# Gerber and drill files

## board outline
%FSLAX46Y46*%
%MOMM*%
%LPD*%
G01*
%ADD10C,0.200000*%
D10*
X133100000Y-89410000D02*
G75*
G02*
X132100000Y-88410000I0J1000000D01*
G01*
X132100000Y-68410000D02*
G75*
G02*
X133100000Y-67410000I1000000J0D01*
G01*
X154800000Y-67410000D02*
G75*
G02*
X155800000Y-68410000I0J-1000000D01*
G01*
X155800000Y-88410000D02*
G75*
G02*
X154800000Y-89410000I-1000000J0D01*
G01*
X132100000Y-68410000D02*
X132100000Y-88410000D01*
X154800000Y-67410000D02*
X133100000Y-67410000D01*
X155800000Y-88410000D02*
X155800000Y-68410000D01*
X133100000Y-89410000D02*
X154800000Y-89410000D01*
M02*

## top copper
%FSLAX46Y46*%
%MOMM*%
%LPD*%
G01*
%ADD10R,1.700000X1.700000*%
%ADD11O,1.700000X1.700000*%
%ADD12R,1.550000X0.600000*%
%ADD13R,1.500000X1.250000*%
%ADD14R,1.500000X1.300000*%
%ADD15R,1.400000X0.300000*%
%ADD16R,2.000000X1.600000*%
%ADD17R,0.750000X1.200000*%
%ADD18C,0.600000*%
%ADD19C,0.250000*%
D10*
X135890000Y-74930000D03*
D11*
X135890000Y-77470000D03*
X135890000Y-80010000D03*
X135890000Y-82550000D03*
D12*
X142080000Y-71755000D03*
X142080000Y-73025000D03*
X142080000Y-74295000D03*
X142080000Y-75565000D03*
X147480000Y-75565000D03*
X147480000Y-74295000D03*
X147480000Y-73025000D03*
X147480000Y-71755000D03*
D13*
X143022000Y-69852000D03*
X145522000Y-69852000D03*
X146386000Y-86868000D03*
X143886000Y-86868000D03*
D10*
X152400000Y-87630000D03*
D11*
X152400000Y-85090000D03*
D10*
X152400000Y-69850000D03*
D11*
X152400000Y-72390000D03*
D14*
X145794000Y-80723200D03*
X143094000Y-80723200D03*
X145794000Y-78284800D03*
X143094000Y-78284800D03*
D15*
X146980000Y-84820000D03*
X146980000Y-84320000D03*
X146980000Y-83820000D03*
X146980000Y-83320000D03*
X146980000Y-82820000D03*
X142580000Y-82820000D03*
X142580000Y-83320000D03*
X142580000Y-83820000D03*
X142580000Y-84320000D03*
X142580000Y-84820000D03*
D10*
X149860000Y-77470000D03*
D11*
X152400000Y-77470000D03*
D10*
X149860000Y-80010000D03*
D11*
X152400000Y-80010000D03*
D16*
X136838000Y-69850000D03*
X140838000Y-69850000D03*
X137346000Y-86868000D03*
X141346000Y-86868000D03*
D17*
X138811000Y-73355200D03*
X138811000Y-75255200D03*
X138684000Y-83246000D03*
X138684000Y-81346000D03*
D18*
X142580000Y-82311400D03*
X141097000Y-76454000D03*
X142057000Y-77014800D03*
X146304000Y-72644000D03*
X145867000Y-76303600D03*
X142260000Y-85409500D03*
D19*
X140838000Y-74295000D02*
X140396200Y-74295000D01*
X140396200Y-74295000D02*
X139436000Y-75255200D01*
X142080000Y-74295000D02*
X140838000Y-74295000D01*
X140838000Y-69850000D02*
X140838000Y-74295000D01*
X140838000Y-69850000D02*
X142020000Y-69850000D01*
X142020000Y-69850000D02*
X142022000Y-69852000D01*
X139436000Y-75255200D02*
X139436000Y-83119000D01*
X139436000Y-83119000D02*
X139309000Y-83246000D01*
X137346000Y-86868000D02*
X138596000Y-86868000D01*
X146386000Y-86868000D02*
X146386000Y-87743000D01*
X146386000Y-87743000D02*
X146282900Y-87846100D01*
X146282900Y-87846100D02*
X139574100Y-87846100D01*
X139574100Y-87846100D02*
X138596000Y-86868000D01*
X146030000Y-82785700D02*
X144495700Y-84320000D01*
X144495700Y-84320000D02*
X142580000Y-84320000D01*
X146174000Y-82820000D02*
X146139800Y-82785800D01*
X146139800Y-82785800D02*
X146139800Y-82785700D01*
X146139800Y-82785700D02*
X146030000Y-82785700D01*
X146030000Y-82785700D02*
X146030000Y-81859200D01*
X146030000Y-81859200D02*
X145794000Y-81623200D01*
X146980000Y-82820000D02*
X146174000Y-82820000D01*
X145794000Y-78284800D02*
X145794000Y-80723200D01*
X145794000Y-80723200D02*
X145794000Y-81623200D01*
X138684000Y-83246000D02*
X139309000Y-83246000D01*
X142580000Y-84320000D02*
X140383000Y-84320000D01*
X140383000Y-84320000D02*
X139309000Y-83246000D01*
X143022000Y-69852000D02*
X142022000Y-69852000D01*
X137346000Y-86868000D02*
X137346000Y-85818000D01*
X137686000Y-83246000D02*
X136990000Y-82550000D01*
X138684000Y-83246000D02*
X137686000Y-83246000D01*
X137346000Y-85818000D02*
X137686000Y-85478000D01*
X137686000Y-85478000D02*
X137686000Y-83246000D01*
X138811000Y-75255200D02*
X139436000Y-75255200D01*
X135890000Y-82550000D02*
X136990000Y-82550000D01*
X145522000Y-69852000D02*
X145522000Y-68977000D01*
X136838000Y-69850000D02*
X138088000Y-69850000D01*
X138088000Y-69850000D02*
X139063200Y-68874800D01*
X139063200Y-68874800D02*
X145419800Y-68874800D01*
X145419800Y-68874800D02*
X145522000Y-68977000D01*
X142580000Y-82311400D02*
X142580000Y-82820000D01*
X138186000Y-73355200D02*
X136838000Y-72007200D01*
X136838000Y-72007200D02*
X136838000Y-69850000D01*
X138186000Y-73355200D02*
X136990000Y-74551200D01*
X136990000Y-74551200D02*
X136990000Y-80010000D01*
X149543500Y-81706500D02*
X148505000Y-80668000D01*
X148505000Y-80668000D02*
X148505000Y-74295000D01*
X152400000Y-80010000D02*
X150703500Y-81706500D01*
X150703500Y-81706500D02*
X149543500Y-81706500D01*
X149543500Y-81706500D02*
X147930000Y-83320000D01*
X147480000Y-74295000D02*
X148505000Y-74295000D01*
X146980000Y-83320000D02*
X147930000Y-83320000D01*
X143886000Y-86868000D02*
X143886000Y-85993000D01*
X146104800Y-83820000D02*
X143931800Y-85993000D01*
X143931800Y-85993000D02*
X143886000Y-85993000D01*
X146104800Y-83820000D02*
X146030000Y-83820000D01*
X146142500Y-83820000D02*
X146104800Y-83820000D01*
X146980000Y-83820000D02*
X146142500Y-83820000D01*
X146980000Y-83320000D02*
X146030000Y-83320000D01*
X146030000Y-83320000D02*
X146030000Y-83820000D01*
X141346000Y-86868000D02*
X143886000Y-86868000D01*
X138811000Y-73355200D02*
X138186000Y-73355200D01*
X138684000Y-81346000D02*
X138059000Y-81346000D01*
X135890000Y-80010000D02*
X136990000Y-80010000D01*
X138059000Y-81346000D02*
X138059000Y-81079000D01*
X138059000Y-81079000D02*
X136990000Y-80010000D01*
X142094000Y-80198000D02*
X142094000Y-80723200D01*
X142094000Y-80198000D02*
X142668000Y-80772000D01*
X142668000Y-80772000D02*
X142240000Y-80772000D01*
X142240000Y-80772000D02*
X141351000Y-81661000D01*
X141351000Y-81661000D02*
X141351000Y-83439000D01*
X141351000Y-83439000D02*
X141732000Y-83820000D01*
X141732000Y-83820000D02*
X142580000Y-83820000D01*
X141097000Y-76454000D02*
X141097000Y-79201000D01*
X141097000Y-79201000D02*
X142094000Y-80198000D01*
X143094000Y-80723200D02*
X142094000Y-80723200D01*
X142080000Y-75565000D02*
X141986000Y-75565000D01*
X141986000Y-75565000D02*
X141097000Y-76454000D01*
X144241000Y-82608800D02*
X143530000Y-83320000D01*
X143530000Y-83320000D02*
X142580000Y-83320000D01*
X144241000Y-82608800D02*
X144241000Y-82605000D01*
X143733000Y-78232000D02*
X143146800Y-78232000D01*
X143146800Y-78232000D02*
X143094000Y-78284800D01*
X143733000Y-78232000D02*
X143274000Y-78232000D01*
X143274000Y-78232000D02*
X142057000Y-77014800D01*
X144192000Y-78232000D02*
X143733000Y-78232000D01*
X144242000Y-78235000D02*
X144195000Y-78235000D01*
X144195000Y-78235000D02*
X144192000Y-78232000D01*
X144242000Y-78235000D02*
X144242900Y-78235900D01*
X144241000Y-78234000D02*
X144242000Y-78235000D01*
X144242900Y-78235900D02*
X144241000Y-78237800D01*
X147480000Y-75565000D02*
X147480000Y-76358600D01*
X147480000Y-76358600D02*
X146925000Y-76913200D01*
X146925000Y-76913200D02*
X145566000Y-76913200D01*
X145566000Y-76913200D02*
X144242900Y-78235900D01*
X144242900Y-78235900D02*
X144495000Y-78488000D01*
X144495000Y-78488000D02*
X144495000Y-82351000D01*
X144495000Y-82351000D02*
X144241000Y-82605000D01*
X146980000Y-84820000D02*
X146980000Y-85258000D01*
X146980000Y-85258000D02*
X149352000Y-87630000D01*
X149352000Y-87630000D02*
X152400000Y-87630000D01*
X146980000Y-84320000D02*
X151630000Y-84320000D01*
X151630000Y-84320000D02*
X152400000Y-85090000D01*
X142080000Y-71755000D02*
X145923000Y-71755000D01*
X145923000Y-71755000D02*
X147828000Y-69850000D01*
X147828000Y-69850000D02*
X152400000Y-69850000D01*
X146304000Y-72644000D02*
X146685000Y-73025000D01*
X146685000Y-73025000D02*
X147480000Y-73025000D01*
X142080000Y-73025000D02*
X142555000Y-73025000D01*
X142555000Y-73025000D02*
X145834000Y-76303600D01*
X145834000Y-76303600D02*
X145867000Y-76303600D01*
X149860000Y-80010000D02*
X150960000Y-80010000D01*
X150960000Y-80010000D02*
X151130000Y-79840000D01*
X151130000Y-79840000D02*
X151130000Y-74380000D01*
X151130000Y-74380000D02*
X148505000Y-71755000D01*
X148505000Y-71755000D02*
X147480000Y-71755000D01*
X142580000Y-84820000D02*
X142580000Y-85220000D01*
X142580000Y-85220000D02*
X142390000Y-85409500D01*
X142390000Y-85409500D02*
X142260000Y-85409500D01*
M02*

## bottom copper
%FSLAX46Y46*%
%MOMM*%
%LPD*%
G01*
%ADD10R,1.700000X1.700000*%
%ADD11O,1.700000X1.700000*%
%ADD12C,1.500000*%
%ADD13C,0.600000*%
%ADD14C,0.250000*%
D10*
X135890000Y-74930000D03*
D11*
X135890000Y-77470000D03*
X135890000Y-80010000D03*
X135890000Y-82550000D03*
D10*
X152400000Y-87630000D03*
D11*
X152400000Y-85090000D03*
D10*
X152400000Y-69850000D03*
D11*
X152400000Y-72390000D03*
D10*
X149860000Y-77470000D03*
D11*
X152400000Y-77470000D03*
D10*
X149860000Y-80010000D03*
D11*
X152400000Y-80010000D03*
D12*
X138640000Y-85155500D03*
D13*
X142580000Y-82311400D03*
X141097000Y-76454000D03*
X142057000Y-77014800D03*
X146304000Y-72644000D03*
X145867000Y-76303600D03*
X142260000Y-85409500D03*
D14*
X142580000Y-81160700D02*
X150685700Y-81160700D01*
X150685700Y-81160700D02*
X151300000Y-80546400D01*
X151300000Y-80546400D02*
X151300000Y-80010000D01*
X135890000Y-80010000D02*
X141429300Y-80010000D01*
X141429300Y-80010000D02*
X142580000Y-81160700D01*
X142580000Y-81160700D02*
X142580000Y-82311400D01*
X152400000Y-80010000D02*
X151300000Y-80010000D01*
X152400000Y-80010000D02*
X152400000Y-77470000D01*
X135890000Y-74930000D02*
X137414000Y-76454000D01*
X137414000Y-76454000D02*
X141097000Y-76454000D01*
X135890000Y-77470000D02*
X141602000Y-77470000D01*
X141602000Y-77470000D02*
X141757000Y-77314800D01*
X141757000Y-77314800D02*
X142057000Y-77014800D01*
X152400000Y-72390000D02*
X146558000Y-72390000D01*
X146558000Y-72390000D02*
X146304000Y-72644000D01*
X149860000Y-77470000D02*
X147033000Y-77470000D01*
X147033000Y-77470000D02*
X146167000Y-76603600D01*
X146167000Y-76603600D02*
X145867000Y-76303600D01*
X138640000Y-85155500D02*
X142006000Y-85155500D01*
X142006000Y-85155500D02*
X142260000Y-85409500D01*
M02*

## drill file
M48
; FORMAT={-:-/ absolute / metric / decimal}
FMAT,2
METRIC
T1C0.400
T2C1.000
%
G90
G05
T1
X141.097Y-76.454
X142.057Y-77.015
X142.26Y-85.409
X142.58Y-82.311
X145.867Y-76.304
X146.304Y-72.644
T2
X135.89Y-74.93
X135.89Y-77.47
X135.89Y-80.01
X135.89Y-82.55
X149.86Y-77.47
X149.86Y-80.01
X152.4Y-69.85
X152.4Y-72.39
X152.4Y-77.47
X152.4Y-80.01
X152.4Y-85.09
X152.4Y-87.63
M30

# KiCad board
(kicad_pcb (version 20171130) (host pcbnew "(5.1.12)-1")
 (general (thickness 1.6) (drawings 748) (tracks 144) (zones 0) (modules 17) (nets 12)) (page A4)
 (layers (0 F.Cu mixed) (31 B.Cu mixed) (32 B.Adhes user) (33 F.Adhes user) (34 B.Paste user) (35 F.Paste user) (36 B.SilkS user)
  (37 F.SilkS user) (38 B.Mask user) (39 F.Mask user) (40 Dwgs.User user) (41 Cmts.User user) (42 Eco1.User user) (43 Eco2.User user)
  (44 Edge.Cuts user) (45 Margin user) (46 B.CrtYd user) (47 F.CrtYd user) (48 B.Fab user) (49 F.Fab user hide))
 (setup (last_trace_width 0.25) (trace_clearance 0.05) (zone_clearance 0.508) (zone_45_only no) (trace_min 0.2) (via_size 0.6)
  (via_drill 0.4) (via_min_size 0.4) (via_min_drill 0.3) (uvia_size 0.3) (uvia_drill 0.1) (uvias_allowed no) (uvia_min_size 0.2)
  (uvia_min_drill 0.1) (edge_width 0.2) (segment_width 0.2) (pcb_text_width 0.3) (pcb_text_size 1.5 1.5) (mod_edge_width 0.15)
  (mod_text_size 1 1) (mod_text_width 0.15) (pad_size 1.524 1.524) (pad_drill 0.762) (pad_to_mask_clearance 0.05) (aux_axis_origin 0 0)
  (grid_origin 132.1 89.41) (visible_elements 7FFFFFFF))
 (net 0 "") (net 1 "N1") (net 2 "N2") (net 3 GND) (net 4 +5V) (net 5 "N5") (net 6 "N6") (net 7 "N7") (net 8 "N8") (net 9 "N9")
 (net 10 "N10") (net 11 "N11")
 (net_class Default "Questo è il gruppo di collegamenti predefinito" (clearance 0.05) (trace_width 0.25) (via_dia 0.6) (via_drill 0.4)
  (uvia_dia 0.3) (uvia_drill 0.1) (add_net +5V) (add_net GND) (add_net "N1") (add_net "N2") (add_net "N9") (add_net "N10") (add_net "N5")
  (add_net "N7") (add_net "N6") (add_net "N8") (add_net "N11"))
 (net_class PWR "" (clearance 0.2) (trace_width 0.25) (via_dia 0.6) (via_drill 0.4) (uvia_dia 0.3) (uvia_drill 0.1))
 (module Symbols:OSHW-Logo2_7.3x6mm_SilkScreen (layer B.Cu) (at 143.784 79.4024 180)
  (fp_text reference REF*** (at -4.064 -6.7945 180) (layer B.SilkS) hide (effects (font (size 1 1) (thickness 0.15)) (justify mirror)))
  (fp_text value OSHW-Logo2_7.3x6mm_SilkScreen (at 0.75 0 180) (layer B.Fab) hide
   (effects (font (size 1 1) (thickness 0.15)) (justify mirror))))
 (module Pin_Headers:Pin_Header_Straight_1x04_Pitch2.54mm (layer F.Cu) (at 135.89 74.93)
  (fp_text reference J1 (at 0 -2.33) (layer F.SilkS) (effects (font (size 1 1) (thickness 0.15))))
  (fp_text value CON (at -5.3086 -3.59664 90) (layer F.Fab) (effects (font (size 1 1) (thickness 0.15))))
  (pad 1 thru_hole rect (at 0 0) (size 1.7 1.7) (drill 1) (layers *.Cu *.Mask) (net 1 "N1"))
  (pad 2 thru_hole oval (at 0 2.54) (size 1.7 1.7) (drill 1) (layers *.Cu *.Mask) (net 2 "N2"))
  (pad 3 thru_hole oval (at 0 5.08) (size 1.7 1.7) (drill 1) (layers *.Cu *.Mask) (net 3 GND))
  (pad 4 thru_hole oval (at 0 7.62) (size 1.7 1.7) (drill 1) (layers *.Cu *.Mask) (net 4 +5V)))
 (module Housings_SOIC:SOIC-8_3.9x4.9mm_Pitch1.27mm (layer F.Cu) (at 144.78 73.66)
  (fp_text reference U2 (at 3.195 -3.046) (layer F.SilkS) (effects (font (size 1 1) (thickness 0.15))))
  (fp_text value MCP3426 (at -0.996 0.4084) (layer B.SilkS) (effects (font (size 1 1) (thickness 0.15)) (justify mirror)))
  (pad 1 smd rect (at -2.7 -1.905) (size 1.55 0.6) (layers F.Cu F.Paste F.Mask) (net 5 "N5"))
  (pad 2 smd rect (at -2.7 -0.635) (size 1.55 0.6) (layers F.Cu F.Paste F.Mask) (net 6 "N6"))
  (pad 3 smd rect (at -2.7 0.635) (size 1.55 0.6) (layers F.Cu F.Paste F.Mask) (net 4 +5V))
  (pad 4 smd rect (at -2.7 1.905) (size 1.55 0.6) (layers F.Cu F.Paste F.Mask) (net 1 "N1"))
  (pad 5 smd rect (at 2.7 1.905) (size 1.55 0.6) (layers F.Cu F.Paste F.Mask) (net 2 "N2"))
  (pad 6 smd rect (at 2.7 0.635) (size 1.55 0.6) (layers F.Cu F.Paste F.Mask) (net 3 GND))
  (pad 7 smd rect (at 2.7 -0.635) (size 1.55 0.6) (layers F.Cu F.Paste F.Mask) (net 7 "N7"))
  (pad 8 smd rect (at 2.7 -1.905) (size 1.55 0.6) (layers F.Cu F.Paste F.Mask) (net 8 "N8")))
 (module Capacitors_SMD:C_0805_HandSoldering (layer F.Cu) (at 144.272 69.852)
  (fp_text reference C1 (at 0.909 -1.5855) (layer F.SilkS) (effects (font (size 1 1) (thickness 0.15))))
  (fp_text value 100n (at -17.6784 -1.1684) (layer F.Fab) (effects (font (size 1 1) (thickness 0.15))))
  (pad 1 smd rect (at -1.25 0) (size 1.5 1.25) (layers F.Cu F.Paste F.Mask) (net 4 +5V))
  (pad 2 smd rect (at 1.25 0) (size 1.5 1.25) (layers F.Cu F.Paste F.Mask) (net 3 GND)))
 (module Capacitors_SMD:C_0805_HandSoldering (layer F.Cu) (at 145.136 86.868 180)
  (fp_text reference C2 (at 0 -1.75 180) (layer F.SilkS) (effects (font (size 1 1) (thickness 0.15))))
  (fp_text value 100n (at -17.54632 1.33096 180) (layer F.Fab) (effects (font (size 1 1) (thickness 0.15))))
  (pad 1 smd rect (at -1.25 0 180) (size 1.5 1.25) (layers F.Cu F.Paste F.Mask) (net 4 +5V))
  (pad 2 smd rect (at 1.25 0 180) (size 1.5 1.25) (layers F.Cu F.Paste F.Mask) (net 3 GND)))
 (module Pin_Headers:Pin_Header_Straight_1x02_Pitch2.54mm (layer F.Cu) (at 152.4 87.63 180)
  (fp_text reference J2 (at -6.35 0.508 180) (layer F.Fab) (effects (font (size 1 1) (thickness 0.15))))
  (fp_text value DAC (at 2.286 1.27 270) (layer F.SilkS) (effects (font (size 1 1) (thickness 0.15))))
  (pad 1 thru_hole rect (at 0 0 180) (size 1.7 1.7) (drill 1) (layers *.Cu *.Mask) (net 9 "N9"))
  (pad 2 thru_hole oval (at 0 2.54 180) (size 1.7 1.7) (drill 1) (layers *.Cu *.Mask) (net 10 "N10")))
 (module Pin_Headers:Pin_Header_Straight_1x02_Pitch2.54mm (layer F.Cu) (at 152.4 69.85)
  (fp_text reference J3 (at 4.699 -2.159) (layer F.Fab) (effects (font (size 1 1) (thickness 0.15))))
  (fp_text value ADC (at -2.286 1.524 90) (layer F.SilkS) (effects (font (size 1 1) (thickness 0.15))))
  (pad 1 thru_hole rect (at 0 0) (size 1.7 1.7) (drill 1) (layers *.Cu *.Mask) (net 5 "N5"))
  (pad 2 thru_hole oval (at 0 2.54) (size 1.7 1.7) (drill 1) (layers *.Cu *.Mask) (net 7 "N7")))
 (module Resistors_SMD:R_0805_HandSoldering (layer F.Cu) (at 144.444 80.7232 180)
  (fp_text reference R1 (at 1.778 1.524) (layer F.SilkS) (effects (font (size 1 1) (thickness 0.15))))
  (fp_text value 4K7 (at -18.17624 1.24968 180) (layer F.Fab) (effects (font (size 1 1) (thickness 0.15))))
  (pad 1 smd rect (at -1.35 0 180) (size 1.5 1.3) (layers F.Cu F.Paste F.Mask) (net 4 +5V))
  (pad 2 smd rect (at 1.35 0 180) (size 1.5 1.3) (layers F.Cu F.Paste F.Mask) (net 1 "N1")))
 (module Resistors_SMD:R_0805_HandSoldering (layer F.Cu) (at 144.444 78.2848 180)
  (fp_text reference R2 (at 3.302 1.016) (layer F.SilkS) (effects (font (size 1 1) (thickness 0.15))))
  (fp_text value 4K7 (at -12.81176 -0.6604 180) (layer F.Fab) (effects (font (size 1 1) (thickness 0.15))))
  (pad 1 smd rect (at -1.35 0 180) (size 1.5 1.3) (layers F.Cu F.Paste F.Mask) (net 4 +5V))
  (pad 2 smd rect (at 1.35 0 180) (size 1.5 1.3) (layers F.Cu F.Paste F.Mask) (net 2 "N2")))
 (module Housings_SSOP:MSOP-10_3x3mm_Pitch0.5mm (layer F.Cu) (at 144.78 83.82 180)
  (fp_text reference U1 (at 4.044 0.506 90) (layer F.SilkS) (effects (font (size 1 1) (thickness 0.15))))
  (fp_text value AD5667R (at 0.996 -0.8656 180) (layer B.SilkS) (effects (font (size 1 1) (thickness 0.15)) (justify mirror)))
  (pad 1 smd rect (at -2.2 -1 180) (size 1.4 0.3) (layers F.Cu F.Paste F.Mask) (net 9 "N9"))
  (pad 2 smd rect (at -2.2 -0.5 180) (size 1.4 0.3) (layers F.Cu F.Paste F.Mask) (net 10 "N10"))
  (pad 3 smd rect (at -2.2 0 180) (size 1.4 0.3) (layers F.Cu F.Paste F.Mask) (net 3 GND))
  (pad 4 smd rect (at -2.2 0.5 180) (size 1.4 0.3) (layers F.Cu F.Paste F.Mask) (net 3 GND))
  (pad 5 smd rect (at -2.2 1 180) (size 1.4 0.3) (layers F.Cu F.Paste F.Mask) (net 4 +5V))
  (pad 6 smd rect (at 2.2 1 180) (size 1.4 0.3) (layers F.Cu F.Paste F.Mask) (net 3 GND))
  (pad 7 smd rect (at 2.2 0.5 180) (size 1.4 0.3) (layers F.Cu F.Paste F.Mask) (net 2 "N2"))
  (pad 8 smd rect (at 2.2 0 180) (size 1.4 0.3) (layers F.Cu F.Paste F.Mask) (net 1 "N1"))
  (pad 9 smd rect (at 2.2 -0.5 180) (size 1.4 0.3) (layers F.Cu F.Paste F.Mask) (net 4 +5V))
  (pad 10 smd rect (at 2.2 -1 180) (size 1.4 0.3) (layers F.Cu F.Paste F.Mask) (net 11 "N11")))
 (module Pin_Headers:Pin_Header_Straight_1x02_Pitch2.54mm (layer F.Cu) (at 149.86 77.47 90)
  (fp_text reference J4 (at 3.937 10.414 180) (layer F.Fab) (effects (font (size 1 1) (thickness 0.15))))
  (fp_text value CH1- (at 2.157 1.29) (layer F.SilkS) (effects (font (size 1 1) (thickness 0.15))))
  (pad 1 thru_hole rect (at 0 0 90) (size 1.7 1.7) (drill 1) (layers *.Cu *.Mask) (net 6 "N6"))
  (pad 2 thru_hole oval (at 0 2.54 90) (size 1.7 1.7) (drill 1) (layers *.Cu *.Mask) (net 3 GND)))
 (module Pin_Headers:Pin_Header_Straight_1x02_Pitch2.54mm (layer F.Cu) (at 149.86 80.01 90)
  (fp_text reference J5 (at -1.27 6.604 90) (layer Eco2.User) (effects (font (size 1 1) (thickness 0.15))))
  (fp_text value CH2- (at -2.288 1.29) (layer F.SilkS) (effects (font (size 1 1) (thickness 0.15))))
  (pad 1 thru_hole rect (at 0 0 90) (size 1.7 1.7) (drill 1) (layers *.Cu *.Mask) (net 8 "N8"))
  (pad 2 thru_hole oval (at 0 2.54 90) (size 1.7 1.7) (drill 1) (layers *.Cu *.Mask) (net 3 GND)))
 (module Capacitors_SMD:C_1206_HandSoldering (layer F.Cu) (at 138.838 69.85 180)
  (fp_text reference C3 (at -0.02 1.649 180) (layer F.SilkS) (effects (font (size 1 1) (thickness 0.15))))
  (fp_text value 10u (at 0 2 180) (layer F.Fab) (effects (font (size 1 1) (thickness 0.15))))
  (pad 2 smd rect (at 2 0 180) (size 2 1.6) (layers F.Cu F.Paste F.Mask) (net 3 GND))
  (pad 1 smd rect (at -2 0 180) (size 2 1.6) (layers F.Cu F.Paste F.Mask) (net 4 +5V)))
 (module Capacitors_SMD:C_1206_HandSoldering (layer F.Cu) (at 139.346 86.868)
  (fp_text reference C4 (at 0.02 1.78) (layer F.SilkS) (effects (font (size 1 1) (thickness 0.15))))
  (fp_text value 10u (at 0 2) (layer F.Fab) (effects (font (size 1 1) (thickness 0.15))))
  (pad 1 smd rect (at -2 0) (size 2 1.6) (layers F.Cu F.Paste F.Mask) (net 4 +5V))
  (pad 2 smd rect (at 2 0) (size 2 1.6) (layers F.Cu F.Paste F.Mask) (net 3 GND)))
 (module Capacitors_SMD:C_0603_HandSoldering (layer F.Cu) (at 138.811 74.3052 90)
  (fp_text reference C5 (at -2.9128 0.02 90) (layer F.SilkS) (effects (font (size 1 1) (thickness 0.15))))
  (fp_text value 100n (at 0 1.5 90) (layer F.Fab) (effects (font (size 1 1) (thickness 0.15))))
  (pad 2 smd rect (at 0.95 0 90) (size 1.2 0.75) (layers F.Cu F.Paste F.Mask) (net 3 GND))
  (pad 1 smd rect (at -0.95 0 90) (size 1.2 0.75) (layers F.Cu F.Paste F.Mask) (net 4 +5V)))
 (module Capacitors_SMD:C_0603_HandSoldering (layer F.Cu) (at 138.684 82.296 90)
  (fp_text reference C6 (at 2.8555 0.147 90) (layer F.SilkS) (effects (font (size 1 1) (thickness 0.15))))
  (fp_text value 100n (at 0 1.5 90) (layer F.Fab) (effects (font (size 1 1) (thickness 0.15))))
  (pad 1 smd rect (at -0.95 0 90) (size 1.2 0.75) (layers F.Cu F.Paste F.Mask) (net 4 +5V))
  (pad 2 smd rect (at 0.95 0 90) (size 1.2 0.75) (layers F.Cu F.Paste F.Mask) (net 3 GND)))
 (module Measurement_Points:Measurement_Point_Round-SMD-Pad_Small (layer B.Cu) (at 138.64 85.1555)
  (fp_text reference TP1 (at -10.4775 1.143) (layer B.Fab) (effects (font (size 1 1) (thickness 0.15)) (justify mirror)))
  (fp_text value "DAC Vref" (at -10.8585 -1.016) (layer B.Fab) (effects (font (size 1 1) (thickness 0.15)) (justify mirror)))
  (pad 1 smd circle (at 0 0) (size 1.5 1.5) (layers B.Cu B.Mask) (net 11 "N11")))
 (gr_arc (start 133.1 88.41) (end 132.1 88.41) (angle -90) (layer Edge.Cuts) (width 0.2))
 (gr_arc (start 133.1 68.41) (end 133.1 67.41) (angle -90) (layer Edge.Cuts) (width 0.2))
 (gr_arc (start 154.8 68.41) (end 155.8 68.41) (angle -90) (layer Edge.Cuts) (width 0.2))
 (gr_arc (start 154.8 88.41) (end 154.8 89.41) (angle -90) (layer Edge.Cuts) (width 0.2))
 (gr_line (start 132.1 68.41) (end 132.1 88.41) (layer Edge.Cuts) (width 0.2))
 (gr_line (start 154.8 67.41) (end 133.1 67.41) (layer Edge.Cuts) (width 0.2))
 (gr_line (start 155.8 88.41) (end 155.8 68.41) (layer Edge.Cuts) (width 0.2))
 (gr_line (start 133.1 89.41) (end 154.8 89.41) (layer Edge.Cuts) (width 0.2))
 (segment (start 140.838 74.295) (end 140.3962 74.295) (width 0.25) (layer F.Cu) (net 4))
 (segment (start 140.3962 74.295) (end 139.436 75.2552) (width 0.25) (layer F.Cu) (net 4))
 (segment (start 142.08 74.295) (end 140.838 74.295) (width 0.25) (layer F.Cu) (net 4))
 (segment (start 140.838 69.85) (end 140.838 74.295) (width 0.25) (layer F.Cu) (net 4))
 (segment (start 140.838 69.85) (end 142.02 69.85) (width 0.25) (layer F.Cu) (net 4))
 (segment (start 142.02 69.85) (end 142.022 69.852) (width 0.25) (layer F.Cu) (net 4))
 (segment (start 139.436 75.2552) (end 139.436 83.119) (width 0.25) (layer F.Cu) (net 4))
 (segment (start 139.436 83.119) (end 139.309 83.246) (width 0.25) (layer F.Cu) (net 4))
 (segment (start 137.346 86.868) (end 138.596 86.868) (width 0.25) (layer F.Cu) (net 4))
 (segment (start 146.386 86.868) (end 146.386 87.743) (width 0.25) (layer F.Cu) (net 4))
 (segment (start 146.386 87.743) (end 146.2829 87.8461) (width 0.25) (layer F.Cu) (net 4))
 (segment (start 146.2829 87.8461) (end 139.5741 87.8461) (width 0.25) (layer F.Cu) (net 4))
 (segment (start 139.5741 87.8461) (end 138.596 86.868) (width 0.25) (layer F.Cu) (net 4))
 (segment (start 146.03 82.7857) (end 144.4957 84.32) (width 0.25) (layer F.Cu) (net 4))
 (segment (start 144.4957 84.32) (end 142.58 84.32) (width 0.25) (layer F.Cu) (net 4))
 (segment (start 146.174 82.82) (end 146.1398 82.7858) (width 0.25) (layer F.Cu) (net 4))
 (segment (start 146.1398 82.7858) (end 146.1398 82.7857) (width 0.25) (layer F.Cu) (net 4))
 (segment (start 146.1398 82.7857) (end 146.03 82.7857) (width 0.25) (layer F.Cu) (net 4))
 (segment (start 146.03 82.7857) (end 146.03 81.8592) (width 0.25) (layer F.Cu) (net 4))
 (segment (start 146.03 81.8592) (end 145.794 81.6232) (width 0.25) (layer F.Cu) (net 4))
 (segment (start 146.98 82.82) (end 146.174 82.82) (width 0.25) (layer F.Cu) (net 4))
 (segment (start 145.794 78.2848) (end 145.794 80.7232) (width 0.25) (layer F.Cu) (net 4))
 (segment (start 145.794 80.7232) (end 145.794 81.6232) (width 0.25) (layer F.Cu) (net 4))
 (segment (start 138.684 83.246) (end 139.309 83.246) (width 0.25) (layer F.Cu) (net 4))
 (segment (start 142.58 84.32) (end 140.383 84.32) (width 0.25) (layer F.Cu) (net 4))
 (segment (start 140.383 84.32) (end 139.309 83.246) (width 0.25) (layer F.Cu) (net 4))
 (segment (start 143.022 69.852) (end 142.022 69.852) (width 0.25) (layer F.Cu) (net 4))
 (segment (start 137.346 86.868) (end 137.346 85.818) (width 0.25) (layer F.Cu) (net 4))
 (segment (start 137.686 83.246) (end 136.99 82.55) (width 0.25) (layer F.Cu) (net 4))
 (segment (start 138.684 83.246) (end 137.686 83.246) (width 0.25) (layer F.Cu) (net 4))
 (segment (start 137.346 85.818) (end 137.686 85.478) (width 0.25) (layer F.Cu) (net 4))
 (segment (start 137.686 85.478) (end 137.686 83.246) (width 0.25) (layer F.Cu) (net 4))
 (segment (start 138.811 75.2552) (end 139.436 75.2552) (width 0.25) (layer F.Cu) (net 4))
 (segment (start 135.89 82.55) (end 136.99 82.55) (width 0.25) (layer F.Cu) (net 4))
 (segment (start 142.58 81.1607) (end 150.6857 81.1607) (width 0.25) (layer B.Cu) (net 3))
 (segment (start 150.6857 81.1607) (end 151.3 80.5464) (width 0.25) (layer B.Cu) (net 3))
 (segment (start 151.3 80.5464) (end 151.3 80.01) (width 0.25) (layer B.Cu) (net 3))
 (segment (start 135.89 80.01) (end 141.4293 80.01) (width 0.25) (layer B.Cu) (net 3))
 (segment (start 141.4293 80.01) (end 142.58 81.1607) (width 0.25) (layer B.Cu) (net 3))
 (segment (start 142.58 81.1607) (end 142.58 82.3114) (width 0.25) (layer B.Cu) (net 3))
 (segment (start 152.4 80.01) (end 151.3 80.01) (width 0.25) (layer B.Cu) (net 3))
 (segment (start 145.522 69.852) (end 145.522 68.977) (width 0.25) (layer F.Cu) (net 3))
 (segment (start 136.838 69.85) (end 138.088 69.85) (width 0.25) (layer F.Cu) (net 3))
 (segment (start 138.088 69.85) (end 139.0632 68.8748) (width 0.25) (layer F.Cu) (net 3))
 (segment (start 139.0632 68.8748) (end 145.4198 68.8748) (width 0.25) (layer F.Cu) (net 3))
 (segment (start 145.4198 68.8748) (end 145.522 68.977) (width 0.25) (layer F.Cu) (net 3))
 (segment (start 142.58 82.3114) (end 142.58 82.82) (width 0.25) (layer F.Cu) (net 3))
 (segment (start 138.186 73.3552) (end 136.838 72.0072) (width 0.25) (layer F.Cu) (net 3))
 (segment (start 136.838 72.0072) (end 136.838 69.85) (width 0.25) (layer F.Cu) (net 3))
 (segment (start 138.186 73.3552) (end 136.99 74.5512) (width 0.25) (layer F.Cu) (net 3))
 (segment (start 136.99 74.5512) (end 136.99 80.01) (width 0.25) (layer F.Cu) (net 3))
 (segment (start 149.5435 81.7065) (end 148.505 80.668) (width 0.25) (layer F.Cu) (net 3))
 (segment (start 148.505 80.668) (end 148.505 74.295) (width 0.25) (layer F.Cu) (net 3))
 (segment (start 152.4 80.01) (end 150.7035 81.7065) (width 0.25) (layer F.Cu) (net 3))
 (segment (start 150.7035 81.7065) (end 149.5435 81.7065) (width 0.25) (layer F.Cu) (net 3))
 (segment (start 149.5435 81.7065) (end 147.93 83.32) (width 0.25) (layer F.Cu) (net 3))
 (segment (start 147.48 74.295) (end 148.505 74.295) (width 0.25) (layer F.Cu) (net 3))
 (segment (start 146.98 83.32) (end 147.93 83.32) (width 0.25) (layer F.Cu) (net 3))
 (segment (start 152.4 80.01) (end 152.4 77.47) (width 0.25) (layer B.Cu) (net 3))
 (segment (start 143.886 86.868) (end 143.886 85.993) (width 0.25) (layer F.Cu) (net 3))
 (segment (start 146.1048 83.82) (end 143.9318 85.993) (width 0.25) (layer F.Cu) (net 3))
 (segment (start 143.9318 85.993) (end 143.886 85.993) (width 0.25) (layer F.Cu) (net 3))
 (segment (start 146.1048 83.82) (end 146.03 83.82) (width 0.25) (layer F.Cu) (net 3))
 (segment (start 146.1425 83.82) (end 146.1048 83.82) (width 0.25) (layer F.Cu) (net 3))
 (segment (start 146.98 83.82) (end 146.1425 83.82) (width 0.25) (layer F.Cu) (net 3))
 (segment (start 146.98 83.32) (end 146.03 83.32) (width 0.25) (layer F.Cu) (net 3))
 (segment (start 146.03 83.32) (end 146.03 83.82) (width 0.25) (layer F.Cu) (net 3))
 (segment (start 141.346 86.868) (end 143.886 86.868) (width 0.25) (layer F.Cu) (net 3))
 (segment (start 138.811 73.3552) (end 138.186 73.3552) (width 0.25) (layer F.Cu) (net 3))
 (segment (start 138.684 81.346) (end 138.059 81.346) (width 0.25) (layer F.Cu) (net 3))
 (segment (start 135.89 80.01) (end 136.99 80.01) (width 0.25) (layer F.Cu) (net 3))
 (segment (start 138.059 81.346) (end 138.059 81.079) (width 0.25) (layer F.Cu) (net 3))
 (segment (start 138.059 81.079) (end 136.99 80.01) (width 0.25) (layer F.Cu) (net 3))
 (via (at 142.58 82.3114) (size 0.6) (layers F.Cu B.Cu) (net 3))
 (segment (start 142.094 80.198) (end 142.094 80.7232) (width 0.25) (layer F.Cu) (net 1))
 (segment (start 142.094 80.198) (end 142.668 80.772) (width 0.25) (layer F.Cu) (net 1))
 (segment (start 142.668 80.772) (end 142.24 80.772) (width 0.25) (layer F.Cu) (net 1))
 (segment (start 142.24 80.772) (end 141.351 81.661) (width 0.25) (layer F.Cu) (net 1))
 (segment (start 141.351 81.661) (end 141.351 83.439) (width 0.25) (layer F.Cu) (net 1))
 (segment (start 141.351 83.439) (end 141.732 83.82) (width 0.25) (layer F.Cu) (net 1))
 (segment (start 141.732 83.82) (end 142.58 83.82) (width 0.25) (layer F.Cu) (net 1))
 (segment (start 141.097 76.454) (end 141.097 79.201) (width 0.25) (layer F.Cu) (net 1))
 (segment (start 141.097 79.201) (end 142.094 80.198) (width 0.25) (layer F.Cu) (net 1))
 (segment (start 143.094 80.7232) (end 142.094 80.7232) (width 0.25) (layer F.Cu) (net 1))
 (segment (start 142.08 75.565) (end 141.986 75.565) (width 0.25) (layer F.Cu) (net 1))
 (segment (start 141.986 75.565) (end 141.097 76.454) (width 0.25) (layer F.Cu) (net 1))
 (segment (start 135.89 74.93) (end 137.414 76.454) (width 0.25) (layer B.Cu) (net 1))
 (segment (start 137.414 76.454) (end 141.097 76.454) (width 0.25) (layer B.Cu) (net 1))
 (via (at 141.097 76.454) (size 0.6) (layers F.Cu B.Cu) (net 1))
 (segment (start 144.241 82.6088) (end 143.53 83.32) (width 0.25) (layer F.Cu) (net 2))
 (segment (start 143.53 83.32) (end 142.58 83.32) (width 0.25) (layer F.Cu) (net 2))
 (segment (start 144.241 82.6088) (end 144.241 82.605) (width 0.25) (layer F.Cu) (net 2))
 (segment (start 143.733 78.232) (end 143.1468 78.232) (width 0.25) (layer F.Cu) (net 2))
 (segment (start 143.1468 78.232) (end 143.094 78.2848) (width 0.25) (layer F.Cu) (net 2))
 (segment (start 143.733 78.232) (end 143.274 78.232) (width 0.25) (layer F.Cu) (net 2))
 (segment (start 143.274 78.232) (end 142.057 77.0148) (width 0.25) (layer F.Cu) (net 2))
 (segment (start 144.192 78.232) (end 143.733 78.232) (width 0.25) (layer F.Cu) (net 2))
 (segment (start 144.242 78.235) (end 144.195 78.235) (width 0.25) (layer F.Cu) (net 2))
 (segment (start 144.195 78.235) (end 144.192 78.232) (width 0.25) (layer F.Cu) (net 2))
 (segment (start 144.242 78.235) (end 144.2429 78.2359) (width 0.25) (layer F.Cu) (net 2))
 (segment (start 144.241 78.234) (end 144.242 78.235) (width 0.25) (layer F.Cu) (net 2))
 (segment (start 144.2429 78.2359) (end 144.241 78.2378) (width 0.25) (layer F.Cu) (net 2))
 (segment (start 147.48 75.565) (end 147.48 76.3586) (width 0.25) (layer F.Cu) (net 2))
 (segment (start 147.48 76.3586) (end 146.925 76.9132) (width 0.25) (layer F.Cu) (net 2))
 (segment (start 146.925 76.9132) (end 145.566 76.9132) (width 0.25) (layer F.Cu) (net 2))
 (segment (start 145.566 76.9132) (end 144.2429 78.2359) (width 0.25) (layer F.Cu) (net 2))
 (segment (start 144.2429 78.2359) (end 144.495 78.488) (width 0.25) (layer F.Cu) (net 2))
 (segment (start 144.495 78.488) (end 144.495 82.351) (width 0.25) (layer F.Cu) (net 2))
 (segment (start 144.495 82.351) (end 144.241 82.605) (width 0.25) (layer F.Cu) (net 2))
 (segment (start 135.89 77.47) (end 141.602 77.47) (width 0.25) (layer B.Cu) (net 2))
 (segment (start 141.602 77.47) (end 141.757 77.3148) (width 0.25) (layer B.Cu) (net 2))
 (segment (start 141.757 77.3148) (end 142.057 77.0148) (width 0.25) (layer B.Cu) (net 2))
 (via (at 142.057 77.0148) (size 0.6) (layers F.Cu B.Cu) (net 2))
 (segment (start 146.98 84.82) (end 146.98 85.258) (width 0.25) (layer F.Cu) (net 9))
 (segment (start 146.98 85.258) (end 149.352 87.63) (width 0.25) (layer F.Cu) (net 9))
 (segment (start 149.352 87.63) (end 152.4 87.63) (width 0.25) (layer F.Cu) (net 9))
 (segment (start 146.98 84.32) (end 151.63 84.32) (width 0.25) (layer F.Cu) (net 10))
 (segment (start 151.63 84.32) (end 152.4 85.09) (width 0.25) (layer F.Cu) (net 10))
 (segment (start 142.08 71.755) (end 145.923 71.755) (width 0.25) (layer F.Cu) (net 5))
 (segment (start 145.923 71.755) (end 147.828 69.85) (width 0.25) (layer F.Cu) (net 5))
 (segment (start 147.828 69.85) (end 152.4 69.85) (width 0.25) (layer F.Cu) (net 5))
 (segment (start 152.4 72.39) (end 146.558 72.39) (width 0.25) (layer B.Cu) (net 7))
 (segment (start 146.558 72.39) (end 146.304 72.644) (width 0.25) (layer B.Cu) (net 7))
 (segment (start 146.304 72.644) (end 146.685 73.025) (width 0.25) (layer F.Cu) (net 7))
 (segment (start 146.685 73.025) (end 147.48 73.025) (width 0.25) (layer F.Cu) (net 7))
 (via (at 146.304 72.644) (size 0.6) (layers F.Cu B.Cu) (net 7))
 (segment (start 142.08 73.025) (end 142.555 73.025) (width 0.25) (layer F.Cu) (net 6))
 (segment (start 142.555 73.025) (end 145.834 76.3036) (width 0.25) (layer F.Cu) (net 6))
 (segment (start 145.834 76.3036) (end 145.867 76.3036) (width 0.25) (layer F.Cu) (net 6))
 (segment (start 149.86 77.47) (end 147.033 77.47) (width 0.25) (layer B.Cu) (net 6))
 (segment (start 147.033 77.47) (end 146.167 76.6036) (width 0.25) (layer B.Cu) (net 6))
 (segment (start 146.167 76.6036) (end 145.867 76.3036) (width 0.25) (layer B.Cu) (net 6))
 (via (at 145.867 76.3036) (size 0.6) (layers F.Cu B.Cu) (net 6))
 (segment (start 149.86 80.01) (end 150.96 80.01) (width 0.25) (layer F.Cu) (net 8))
 (segment (start 150.96 80.01) (end 151.13 79.84) (width 0.25) (layer F.Cu) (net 8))
 (segment (start 151.13 79.84) (end 151.13 74.38) (width 0.25) (layer F.Cu) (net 8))
 (segment (start 151.13 74.38) (end 148.505 71.755) (width 0.25) (layer F.Cu) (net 8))
 (segment (start 148.505 71.755) (end 147.48 71.755) (width 0.25) (layer F.Cu) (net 8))
 (segment (start 142.58 84.82) (end 142.58 85.22) (width 0.25) (layer F.Cu) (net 11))
 (segment (start 142.58 85.22) (end 142.39 85.4095) (width 0.25) (layer F.Cu) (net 11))
 (segment (start 142.39 85.4095) (end 142.26 85.4095) (width 0.25) (layer F.Cu) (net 11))
 (segment (start 138.64 85.1555) (end 142.006 85.1555) (width 0.25) (layer B.Cu) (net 11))
 (segment (start 142.006 85.1555) (end 142.26 85.4095) (width 0.25) (layer B.Cu) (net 11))
 (via (at 142.26 85.4095) (size 0.6) (layers F.Cu B.Cu) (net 11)))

